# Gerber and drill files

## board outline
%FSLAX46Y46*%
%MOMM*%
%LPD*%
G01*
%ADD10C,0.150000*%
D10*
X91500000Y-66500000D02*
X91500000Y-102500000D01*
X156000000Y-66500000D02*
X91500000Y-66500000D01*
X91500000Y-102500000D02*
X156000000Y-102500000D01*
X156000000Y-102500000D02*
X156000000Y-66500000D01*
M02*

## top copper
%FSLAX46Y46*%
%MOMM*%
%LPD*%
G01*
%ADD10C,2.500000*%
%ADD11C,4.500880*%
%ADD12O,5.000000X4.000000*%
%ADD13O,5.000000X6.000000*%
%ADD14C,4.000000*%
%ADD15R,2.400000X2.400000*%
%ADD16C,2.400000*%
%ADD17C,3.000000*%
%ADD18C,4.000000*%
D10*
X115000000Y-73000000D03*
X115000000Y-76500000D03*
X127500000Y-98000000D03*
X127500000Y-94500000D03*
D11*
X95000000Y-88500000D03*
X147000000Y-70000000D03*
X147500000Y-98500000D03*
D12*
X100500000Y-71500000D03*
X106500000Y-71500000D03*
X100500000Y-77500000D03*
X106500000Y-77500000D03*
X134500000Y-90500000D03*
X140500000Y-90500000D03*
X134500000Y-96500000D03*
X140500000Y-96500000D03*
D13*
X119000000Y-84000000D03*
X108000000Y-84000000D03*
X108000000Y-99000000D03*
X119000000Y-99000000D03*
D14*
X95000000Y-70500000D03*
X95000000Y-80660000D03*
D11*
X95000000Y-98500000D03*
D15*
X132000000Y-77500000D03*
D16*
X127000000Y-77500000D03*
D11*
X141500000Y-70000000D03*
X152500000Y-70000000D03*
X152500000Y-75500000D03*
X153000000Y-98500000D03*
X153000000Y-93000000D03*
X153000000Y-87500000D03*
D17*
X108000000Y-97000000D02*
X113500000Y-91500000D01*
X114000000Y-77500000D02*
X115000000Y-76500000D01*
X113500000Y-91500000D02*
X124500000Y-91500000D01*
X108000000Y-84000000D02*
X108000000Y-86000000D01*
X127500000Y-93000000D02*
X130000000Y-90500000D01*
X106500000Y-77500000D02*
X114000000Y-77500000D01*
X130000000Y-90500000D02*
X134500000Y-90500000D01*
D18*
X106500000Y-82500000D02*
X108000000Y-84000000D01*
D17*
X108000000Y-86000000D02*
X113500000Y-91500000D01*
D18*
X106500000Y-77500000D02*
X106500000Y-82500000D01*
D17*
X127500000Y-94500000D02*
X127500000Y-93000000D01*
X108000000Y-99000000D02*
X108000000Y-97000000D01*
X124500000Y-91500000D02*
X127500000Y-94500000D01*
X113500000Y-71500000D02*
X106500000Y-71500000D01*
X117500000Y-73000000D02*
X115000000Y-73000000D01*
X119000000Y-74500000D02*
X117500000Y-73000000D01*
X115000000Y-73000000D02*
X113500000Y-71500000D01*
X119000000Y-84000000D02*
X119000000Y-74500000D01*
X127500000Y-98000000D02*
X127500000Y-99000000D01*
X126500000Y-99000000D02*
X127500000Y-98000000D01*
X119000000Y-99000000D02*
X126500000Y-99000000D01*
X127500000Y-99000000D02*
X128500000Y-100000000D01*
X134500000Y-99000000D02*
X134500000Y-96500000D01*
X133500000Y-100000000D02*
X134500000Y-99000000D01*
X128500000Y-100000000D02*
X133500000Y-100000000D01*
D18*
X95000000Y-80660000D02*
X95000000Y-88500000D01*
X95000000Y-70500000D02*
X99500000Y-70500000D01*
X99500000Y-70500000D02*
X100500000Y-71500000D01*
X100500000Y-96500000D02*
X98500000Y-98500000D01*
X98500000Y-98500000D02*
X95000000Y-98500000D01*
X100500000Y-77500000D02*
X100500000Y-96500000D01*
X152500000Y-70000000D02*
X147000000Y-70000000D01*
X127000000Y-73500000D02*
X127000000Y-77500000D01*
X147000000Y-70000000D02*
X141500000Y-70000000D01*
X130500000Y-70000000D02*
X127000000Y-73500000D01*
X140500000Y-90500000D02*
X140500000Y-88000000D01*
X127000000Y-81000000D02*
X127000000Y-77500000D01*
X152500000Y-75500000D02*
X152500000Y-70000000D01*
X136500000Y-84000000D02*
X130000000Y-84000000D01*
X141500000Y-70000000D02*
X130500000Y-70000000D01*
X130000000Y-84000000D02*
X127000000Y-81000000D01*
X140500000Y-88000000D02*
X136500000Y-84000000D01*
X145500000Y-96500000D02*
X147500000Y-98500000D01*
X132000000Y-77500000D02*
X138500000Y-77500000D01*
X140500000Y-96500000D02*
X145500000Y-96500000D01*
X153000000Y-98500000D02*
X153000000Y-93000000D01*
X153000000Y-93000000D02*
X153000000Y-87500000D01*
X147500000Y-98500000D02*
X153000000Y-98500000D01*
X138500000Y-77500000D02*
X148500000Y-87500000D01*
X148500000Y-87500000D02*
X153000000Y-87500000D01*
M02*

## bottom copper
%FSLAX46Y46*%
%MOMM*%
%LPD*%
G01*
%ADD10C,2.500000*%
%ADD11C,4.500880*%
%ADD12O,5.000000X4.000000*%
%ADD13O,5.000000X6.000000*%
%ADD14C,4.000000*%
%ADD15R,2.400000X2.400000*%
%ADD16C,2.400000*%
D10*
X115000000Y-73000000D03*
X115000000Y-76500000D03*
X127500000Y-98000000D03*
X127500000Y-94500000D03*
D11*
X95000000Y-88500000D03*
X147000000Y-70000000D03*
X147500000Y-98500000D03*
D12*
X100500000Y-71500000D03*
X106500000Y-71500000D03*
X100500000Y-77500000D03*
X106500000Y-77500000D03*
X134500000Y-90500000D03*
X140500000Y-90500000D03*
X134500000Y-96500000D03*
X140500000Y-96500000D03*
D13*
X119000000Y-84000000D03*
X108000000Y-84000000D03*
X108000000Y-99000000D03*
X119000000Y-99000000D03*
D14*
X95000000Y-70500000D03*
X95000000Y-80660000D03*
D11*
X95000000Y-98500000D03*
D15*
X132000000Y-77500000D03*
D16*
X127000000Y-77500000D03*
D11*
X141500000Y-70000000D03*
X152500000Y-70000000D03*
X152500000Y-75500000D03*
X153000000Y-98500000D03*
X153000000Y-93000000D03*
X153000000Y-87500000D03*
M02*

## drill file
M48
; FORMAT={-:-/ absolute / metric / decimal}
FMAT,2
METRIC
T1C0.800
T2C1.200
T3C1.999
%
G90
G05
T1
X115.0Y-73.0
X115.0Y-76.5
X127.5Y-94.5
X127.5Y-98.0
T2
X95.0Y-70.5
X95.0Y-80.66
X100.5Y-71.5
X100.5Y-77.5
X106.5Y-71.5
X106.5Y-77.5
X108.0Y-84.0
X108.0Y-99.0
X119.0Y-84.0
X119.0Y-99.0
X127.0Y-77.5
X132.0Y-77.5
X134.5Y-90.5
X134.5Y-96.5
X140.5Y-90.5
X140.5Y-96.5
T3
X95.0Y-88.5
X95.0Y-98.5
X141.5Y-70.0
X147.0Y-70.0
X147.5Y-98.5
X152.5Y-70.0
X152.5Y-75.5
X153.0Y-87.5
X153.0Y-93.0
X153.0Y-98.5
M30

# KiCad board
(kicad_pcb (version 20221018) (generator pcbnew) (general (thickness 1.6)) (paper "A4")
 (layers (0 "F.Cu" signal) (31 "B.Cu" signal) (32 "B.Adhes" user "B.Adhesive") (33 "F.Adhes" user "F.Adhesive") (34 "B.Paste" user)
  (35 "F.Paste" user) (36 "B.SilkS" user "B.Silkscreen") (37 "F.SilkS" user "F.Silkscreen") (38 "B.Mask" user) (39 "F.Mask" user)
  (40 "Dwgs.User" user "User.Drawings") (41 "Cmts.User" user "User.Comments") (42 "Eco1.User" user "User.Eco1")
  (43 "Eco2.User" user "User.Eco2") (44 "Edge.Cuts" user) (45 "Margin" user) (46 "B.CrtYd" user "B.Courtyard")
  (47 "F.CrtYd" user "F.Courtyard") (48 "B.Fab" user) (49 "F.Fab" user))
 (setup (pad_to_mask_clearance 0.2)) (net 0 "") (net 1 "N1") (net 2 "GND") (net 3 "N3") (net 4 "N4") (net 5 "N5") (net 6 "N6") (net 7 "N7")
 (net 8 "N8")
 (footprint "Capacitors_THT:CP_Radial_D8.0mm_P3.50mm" (layer "F.Cu") (at 115 73 -90)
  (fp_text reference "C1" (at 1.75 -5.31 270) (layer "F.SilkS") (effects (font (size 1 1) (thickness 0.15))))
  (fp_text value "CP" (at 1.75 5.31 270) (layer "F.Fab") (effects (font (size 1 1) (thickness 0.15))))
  (pad "1" thru_hole circle (at 0 0 270) (size 2.5 2.5) (drill 0.8) (layers "*.Cu" "*.Mask") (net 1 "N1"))
  (pad "2" thru_hole circle (at 3.5 0 270) (size 2.5 2.5) (drill 0.8) (layers "*.Cu" "*.Mask") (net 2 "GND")))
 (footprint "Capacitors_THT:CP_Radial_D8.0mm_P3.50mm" (layer "F.Cu") (at 127.5 98 90)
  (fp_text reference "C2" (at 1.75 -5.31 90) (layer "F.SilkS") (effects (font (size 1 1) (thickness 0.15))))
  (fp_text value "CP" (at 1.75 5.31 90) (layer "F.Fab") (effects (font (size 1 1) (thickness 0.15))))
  (pad "1" thru_hole circle (at 0 0 90) (size 2.5 2.5) (drill 0.8) (layers "*.Cu" "*.Mask") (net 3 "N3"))
  (pad "2" thru_hole circle (at 3.5 0 90) (size 2.5 2.5) (drill 0.8) (layers "*.Cu" "*.Mask") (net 2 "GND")))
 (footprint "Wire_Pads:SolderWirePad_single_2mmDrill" (layer "F.Cu") (at 95 88.5)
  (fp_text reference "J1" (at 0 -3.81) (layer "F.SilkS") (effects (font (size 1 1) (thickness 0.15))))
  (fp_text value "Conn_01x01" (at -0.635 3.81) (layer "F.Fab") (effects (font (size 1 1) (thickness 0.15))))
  (pad "1" thru_hole circle (at 0 0) (size 4.50088 4.50088) (drill 1.99898) (layers "*.Cu" "*.Mask") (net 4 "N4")))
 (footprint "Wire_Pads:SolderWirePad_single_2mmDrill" (layer "F.Cu") (at 147 70)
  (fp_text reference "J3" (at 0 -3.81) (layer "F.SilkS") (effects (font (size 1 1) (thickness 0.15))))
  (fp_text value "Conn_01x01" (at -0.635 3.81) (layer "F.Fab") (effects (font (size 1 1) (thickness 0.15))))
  (pad "1" thru_hole circle (at 0 0) (size 4.50088 4.50088) (drill 1.99898) (layers "*.Cu" "*.Mask") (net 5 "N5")))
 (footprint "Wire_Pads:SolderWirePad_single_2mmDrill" (layer "F.Cu") (at 147.5 98.5)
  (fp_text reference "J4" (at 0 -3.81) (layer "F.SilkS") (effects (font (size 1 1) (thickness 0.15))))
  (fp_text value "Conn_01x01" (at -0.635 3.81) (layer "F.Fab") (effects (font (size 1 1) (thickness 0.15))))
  (pad "1" thru_hole circle (at 0 0) (size 4.50088 4.50088) (drill 1.99898) (layers "*.Cu" "*.Mask") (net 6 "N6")))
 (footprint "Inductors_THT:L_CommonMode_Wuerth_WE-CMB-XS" (layer "F.Cu") (at 103.5 74.5)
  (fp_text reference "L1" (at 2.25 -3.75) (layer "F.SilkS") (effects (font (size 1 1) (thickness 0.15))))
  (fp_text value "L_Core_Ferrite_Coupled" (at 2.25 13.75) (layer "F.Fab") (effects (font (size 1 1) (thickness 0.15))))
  (pad "1" thru_hole oval (at -3 -3) (size 5 4) (drill 1.2) (layers "*.Cu" "*.Mask") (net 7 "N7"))
  (pad "2" thru_hole oval (at 3 -3) (size 5 4) (drill 1.2) (layers "*.Cu" "*.Mask") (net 1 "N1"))
  (pad "3" thru_hole oval (at -3 3) (size 5 4) (drill 1.2) (layers "*.Cu" "*.Mask") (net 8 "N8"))
  (pad "4" thru_hole oval (at 3 3) (size 5 4) (drill 1.2) (layers "*.Cu" "*.Mask") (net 2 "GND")))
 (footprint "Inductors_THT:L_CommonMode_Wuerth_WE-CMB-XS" (layer "F.Cu") (at 137.5 93.5)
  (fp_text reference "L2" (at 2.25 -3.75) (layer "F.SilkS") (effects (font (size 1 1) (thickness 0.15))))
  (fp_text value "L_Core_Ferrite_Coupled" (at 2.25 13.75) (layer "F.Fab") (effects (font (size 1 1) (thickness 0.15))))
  (pad "1" thru_hole oval (at -3 -3) (size 5 4) (drill 1.2) (layers "*.Cu" "*.Mask") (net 2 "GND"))
  (pad "2" thru_hole oval (at 3 -3) (size 5 4) (drill 1.2) (layers "*.Cu" "*.Mask") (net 5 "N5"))
  (pad "3" thru_hole oval (at -3 3) (size 5 4) (drill 1.2) (layers "*.Cu" "*.Mask") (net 3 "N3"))
  (pad "4" thru_hole oval (at 3 3) (size 5 4) (drill 1.2) (layers "*.Cu" "*.Mask") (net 6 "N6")))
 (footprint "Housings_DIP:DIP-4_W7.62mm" (layer "F.Cu") (at 113.5 91.5 -90)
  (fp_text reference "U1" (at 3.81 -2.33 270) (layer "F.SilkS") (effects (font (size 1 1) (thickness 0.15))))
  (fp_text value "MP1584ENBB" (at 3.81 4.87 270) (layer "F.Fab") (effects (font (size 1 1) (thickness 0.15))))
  (pad "1" thru_hole oval (at -7.5 -5.5 270) (size 6 5) (drill 1.2) (layers "*.Cu" "*.Mask") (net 1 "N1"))
  (pad "2" thru_hole oval (at -7.5 5.5 270) (size 6 5) (drill 1.2) (layers "*.Cu" "*.Mask") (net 2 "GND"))
  (pad "3" thru_hole oval (at 7.5 5.5 270) (size 6 5) (drill 1.2) (layers "*.Cu" "*.Mask") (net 2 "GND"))
  (pad "4" thru_hole oval (at 7.5 -5.5 270) (size 6 5) (drill 1.2) (layers "*.Cu" "*.Mask") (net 3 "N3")))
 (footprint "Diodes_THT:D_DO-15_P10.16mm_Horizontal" (layer "F.Cu") (at 95 70.5 -90)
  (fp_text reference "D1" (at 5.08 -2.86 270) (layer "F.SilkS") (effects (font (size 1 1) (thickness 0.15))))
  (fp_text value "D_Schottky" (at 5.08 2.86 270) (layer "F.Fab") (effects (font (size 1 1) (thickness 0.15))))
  (pad "1" thru_hole circle (at 0 0 270) (size 4 4) (drill 1.2) (layers "*.Cu" "*.Mask") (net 7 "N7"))
  (pad "2" thru_hole circle (at 10.16 0 270) (size 4 4) (drill 1.2) (layers "*.Cu" "*.Mask") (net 4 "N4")))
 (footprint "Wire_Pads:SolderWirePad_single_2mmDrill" (layer "F.Cu") (at 95 98.5)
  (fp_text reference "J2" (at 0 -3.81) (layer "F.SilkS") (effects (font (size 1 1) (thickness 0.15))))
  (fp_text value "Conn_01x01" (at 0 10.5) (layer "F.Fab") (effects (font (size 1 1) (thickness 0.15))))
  (pad "1" thru_hole circle (at 0 0) (size 4.50088 4.50088) (drill 1.99898) (layers "*.Cu" "*.Mask") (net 8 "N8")))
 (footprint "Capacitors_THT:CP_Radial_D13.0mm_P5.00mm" (layer "F.Cu") (at 132 77.5 180)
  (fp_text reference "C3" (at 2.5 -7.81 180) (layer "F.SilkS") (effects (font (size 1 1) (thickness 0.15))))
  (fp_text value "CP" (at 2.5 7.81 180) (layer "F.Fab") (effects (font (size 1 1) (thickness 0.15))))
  (pad "1" thru_hole rect (at 0 0 180) (size 2.4 2.4) (drill 1.2) (layers "*.Cu" "*.Mask") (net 6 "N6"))
  (pad "2" thru_hole circle (at 5 0 180) (size 2.4 2.4) (drill 1.2) (layers "*.Cu" "*.Mask") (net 5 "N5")))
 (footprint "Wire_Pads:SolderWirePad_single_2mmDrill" (layer "F.Cu") (at 141.5 70)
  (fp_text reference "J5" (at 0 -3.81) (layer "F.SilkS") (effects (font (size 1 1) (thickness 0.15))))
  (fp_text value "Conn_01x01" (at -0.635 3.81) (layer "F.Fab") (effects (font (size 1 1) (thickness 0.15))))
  (pad "1" thru_hole circle (at 0 0) (size 4.50088 4.50088) (drill 1.99898) (layers "*.Cu" "*.Mask") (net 5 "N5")))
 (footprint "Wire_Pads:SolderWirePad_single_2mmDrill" (layer "F.Cu") (at 152.5 70)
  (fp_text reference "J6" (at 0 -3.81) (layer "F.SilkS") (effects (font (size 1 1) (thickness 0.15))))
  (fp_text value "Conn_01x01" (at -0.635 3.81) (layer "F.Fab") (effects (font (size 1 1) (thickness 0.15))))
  (pad "1" thru_hole circle (at 0 0) (size 4.50088 4.50088) (drill 1.99898) (layers "*.Cu" "*.Mask") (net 5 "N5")))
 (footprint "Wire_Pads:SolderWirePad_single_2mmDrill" (layer "F.Cu") (at 152.5 75.5)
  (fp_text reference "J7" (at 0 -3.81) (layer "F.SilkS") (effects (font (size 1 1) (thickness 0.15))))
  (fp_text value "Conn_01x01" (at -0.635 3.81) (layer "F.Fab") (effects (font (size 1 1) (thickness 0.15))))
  (pad "1" thru_hole circle (at 0 0) (size 4.50088 4.50088) (drill 1.99898) (layers "*.Cu" "*.Mask") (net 5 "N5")))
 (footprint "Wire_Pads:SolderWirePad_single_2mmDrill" (layer "F.Cu") (at 153 98.5)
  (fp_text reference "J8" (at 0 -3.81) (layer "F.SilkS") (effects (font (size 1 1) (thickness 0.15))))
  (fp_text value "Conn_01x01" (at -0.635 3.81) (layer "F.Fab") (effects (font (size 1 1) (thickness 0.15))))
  (pad "1" thru_hole circle (at 0 0) (size 4.50088 4.50088) (drill 1.99898) (layers "*.Cu" "*.Mask") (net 6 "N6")))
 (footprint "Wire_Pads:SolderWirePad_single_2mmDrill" (layer "F.Cu") (at 153 93)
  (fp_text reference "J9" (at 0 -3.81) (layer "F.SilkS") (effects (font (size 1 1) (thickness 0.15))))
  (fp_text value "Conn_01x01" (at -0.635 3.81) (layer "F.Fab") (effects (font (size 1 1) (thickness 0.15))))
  (pad "1" thru_hole circle (at 0 0) (size 4.50088 4.50088) (drill 1.99898) (layers "*.Cu" "*.Mask") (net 6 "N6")))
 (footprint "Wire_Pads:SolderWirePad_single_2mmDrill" (layer "F.Cu") (at 153 87.5)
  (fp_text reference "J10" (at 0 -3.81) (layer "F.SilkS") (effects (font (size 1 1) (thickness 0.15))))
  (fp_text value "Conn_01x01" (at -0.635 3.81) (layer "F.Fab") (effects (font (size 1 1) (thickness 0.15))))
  (pad "1" thru_hole circle (at 0 0) (size 4.50088 4.50088) (drill 1.99898) (layers "*.Cu" "*.Mask") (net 6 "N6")))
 (gr_line (start 91.5 66.5) (end 91.5 102.5) (stroke (width 0.15) (type solid)) (layer "Edge.Cuts"))
 (gr_line (start 156 66.5) (end 91.5 66.5) (stroke (width 0.15) (type solid)) (layer "Edge.Cuts"))
 (gr_line (start 91.5 102.5) (end 156 102.5) (stroke (width 0.15) (type solid)) (layer "Edge.Cuts"))
 (gr_line (start 156 102.5) (end 156 66.5) (stroke (width 0.15) (type solid)) (layer "Edge.Cuts"))
 (segment (start 108 97) (end 113.5 91.5) (width 3) (layer "F.Cu") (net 2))
 (segment (start 114 77.5) (end 115 76.5) (width 3) (layer "F.Cu") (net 2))
 (segment (start 113.5 91.5) (end 124.5 91.5) (width 3) (layer "F.Cu") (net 2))
 (segment (start 108 84) (end 108 86) (width 3) (layer "F.Cu") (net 2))
 (segment (start 127.5 93) (end 130 90.5) (width 3) (layer "F.Cu") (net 2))
 (segment (start 106.5 77.5) (end 114 77.5) (width 3) (layer "F.Cu") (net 2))
 (segment (start 130 90.5) (end 134.5 90.5) (width 3) (layer "F.Cu") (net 2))
 (segment (start 106.5 82.5) (end 108 84) (width 4) (layer "F.Cu") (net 2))
 (segment (start 108 86) (end 113.5 91.5) (width 3) (layer "F.Cu") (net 2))
 (segment (start 106.5 77.5) (end 106.5 82.5) (width 4) (layer "F.Cu") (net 2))
 (segment (start 127.5 94.5) (end 127.5 93) (width 3) (layer "F.Cu") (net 2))
 (segment (start 108 99) (end 108 97) (width 3) (layer "F.Cu") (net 2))
 (segment (start 124.5 91.5) (end 127.5 94.5) (width 3) (layer "F.Cu") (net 2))
 (segment (start 113.5 71.5) (end 106.5 71.5) (width 3) (layer "F.Cu") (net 1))
 (segment (start 117.5 73) (end 115 73) (width 3) (layer "F.Cu") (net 1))
 (segment (start 119 74.5) (end 117.5 73) (width 3) (layer "F.Cu") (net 1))
 (segment (start 115 73) (end 113.5 71.5) (width 3) (layer "F.Cu") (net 1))
 (segment (start 119 84) (end 119 74.5) (width 3) (layer "F.Cu") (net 1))
 (segment (start 127.5 98) (end 127.5 99) (width 3) (layer "F.Cu") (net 3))
 (segment (start 126.5 99) (end 127.5 98) (width 3) (layer "F.Cu") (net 3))
 (segment (start 119 99) (end 126.5 99) (width 3) (layer "F.Cu") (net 3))
 (segment (start 127.5 99) (end 128.5 100) (width 3) (layer "F.Cu") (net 3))
 (segment (start 134.5 99) (end 134.5 96.5) (width 3) (layer "F.Cu") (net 3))
 (segment (start 133.5 100) (end 134.5 99) (width 3) (layer "F.Cu") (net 3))
 (segment (start 128.5 100) (end 133.5 100) (width 3) (layer "F.Cu") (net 3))
 (segment (start 95 80.66) (end 95 88.5) (width 4) (layer "F.Cu") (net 4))
 (segment (start 95 70.5) (end 99.5 70.5) (width 4) (layer "F.Cu") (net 7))
 (segment (start 99.5 70.5) (end 100.5 71.5) (width 4) (layer "F.Cu") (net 7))
 (segment (start 100.5 96.5) (end 98.5 98.5) (width 4) (layer "F.Cu") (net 8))
 (segment (start 98.5 98.5) (end 95 98.5) (width 4) (layer "F.Cu") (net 8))
 (segment (start 100.5 77.5) (end 100.5 96.5) (width 4) (layer "F.Cu") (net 8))
 (segment (start 152.5 70) (end 147 70) (width 4) (layer "F.Cu") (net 5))
 (segment (start 127 73.5) (end 127 77.5) (width 4) (layer "F.Cu") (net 5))
 (segment (start 147 70) (end 141.5 70) (width 4) (layer "F.Cu") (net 5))
 (segment (start 130.5 70) (end 127 73.5) (width 4) (layer "F.Cu") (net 5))
 (segment (start 140.5 90.5) (end 140.5 88) (width 4) (layer "F.Cu") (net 5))
 (segment (start 127 81) (end 127 77.5) (width 4) (layer "F.Cu") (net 5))
 (segment (start 152.5 75.5) (end 152.5 70) (width 4) (layer "F.Cu") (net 5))
 (segment (start 136.5 84) (end 130 84) (width 4) (layer "F.Cu") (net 5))
 (segment (start 141.5 70) (end 130.5 70) (width 4) (layer "F.Cu") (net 5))
 (segment (start 130 84) (end 127 81) (width 4) (layer "F.Cu") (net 5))
 (segment (start 140.5 88) (end 136.5 84) (width 4) (layer "F.Cu") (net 5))
 (segment (start 145.5 96.5) (end 147.5 98.5) (width 4) (layer "F.Cu") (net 6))
 (segment (start 132 77.5) (end 138.5 77.5) (width 4) (layer "F.Cu") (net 6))
 (segment (start 140.5 96.5) (end 145.5 96.5) (width 4) (layer "F.Cu") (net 6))
 (segment (start 153 98.5) (end 153 93) (width 4) (layer "F.Cu") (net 6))
 (segment (start 153 93) (end 153 87.5) (width 4) (layer "F.Cu") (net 6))
 (segment (start 147.5 98.5) (end 153 98.5) (width 4) (layer "F.Cu") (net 6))
 (segment (start 138.5 77.5) (end 148.5 87.5) (width 4) (layer "F.Cu") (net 6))
 (segment (start 148.5 87.5) (end 153 87.5) (width 4) (layer "F.Cu") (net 6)))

